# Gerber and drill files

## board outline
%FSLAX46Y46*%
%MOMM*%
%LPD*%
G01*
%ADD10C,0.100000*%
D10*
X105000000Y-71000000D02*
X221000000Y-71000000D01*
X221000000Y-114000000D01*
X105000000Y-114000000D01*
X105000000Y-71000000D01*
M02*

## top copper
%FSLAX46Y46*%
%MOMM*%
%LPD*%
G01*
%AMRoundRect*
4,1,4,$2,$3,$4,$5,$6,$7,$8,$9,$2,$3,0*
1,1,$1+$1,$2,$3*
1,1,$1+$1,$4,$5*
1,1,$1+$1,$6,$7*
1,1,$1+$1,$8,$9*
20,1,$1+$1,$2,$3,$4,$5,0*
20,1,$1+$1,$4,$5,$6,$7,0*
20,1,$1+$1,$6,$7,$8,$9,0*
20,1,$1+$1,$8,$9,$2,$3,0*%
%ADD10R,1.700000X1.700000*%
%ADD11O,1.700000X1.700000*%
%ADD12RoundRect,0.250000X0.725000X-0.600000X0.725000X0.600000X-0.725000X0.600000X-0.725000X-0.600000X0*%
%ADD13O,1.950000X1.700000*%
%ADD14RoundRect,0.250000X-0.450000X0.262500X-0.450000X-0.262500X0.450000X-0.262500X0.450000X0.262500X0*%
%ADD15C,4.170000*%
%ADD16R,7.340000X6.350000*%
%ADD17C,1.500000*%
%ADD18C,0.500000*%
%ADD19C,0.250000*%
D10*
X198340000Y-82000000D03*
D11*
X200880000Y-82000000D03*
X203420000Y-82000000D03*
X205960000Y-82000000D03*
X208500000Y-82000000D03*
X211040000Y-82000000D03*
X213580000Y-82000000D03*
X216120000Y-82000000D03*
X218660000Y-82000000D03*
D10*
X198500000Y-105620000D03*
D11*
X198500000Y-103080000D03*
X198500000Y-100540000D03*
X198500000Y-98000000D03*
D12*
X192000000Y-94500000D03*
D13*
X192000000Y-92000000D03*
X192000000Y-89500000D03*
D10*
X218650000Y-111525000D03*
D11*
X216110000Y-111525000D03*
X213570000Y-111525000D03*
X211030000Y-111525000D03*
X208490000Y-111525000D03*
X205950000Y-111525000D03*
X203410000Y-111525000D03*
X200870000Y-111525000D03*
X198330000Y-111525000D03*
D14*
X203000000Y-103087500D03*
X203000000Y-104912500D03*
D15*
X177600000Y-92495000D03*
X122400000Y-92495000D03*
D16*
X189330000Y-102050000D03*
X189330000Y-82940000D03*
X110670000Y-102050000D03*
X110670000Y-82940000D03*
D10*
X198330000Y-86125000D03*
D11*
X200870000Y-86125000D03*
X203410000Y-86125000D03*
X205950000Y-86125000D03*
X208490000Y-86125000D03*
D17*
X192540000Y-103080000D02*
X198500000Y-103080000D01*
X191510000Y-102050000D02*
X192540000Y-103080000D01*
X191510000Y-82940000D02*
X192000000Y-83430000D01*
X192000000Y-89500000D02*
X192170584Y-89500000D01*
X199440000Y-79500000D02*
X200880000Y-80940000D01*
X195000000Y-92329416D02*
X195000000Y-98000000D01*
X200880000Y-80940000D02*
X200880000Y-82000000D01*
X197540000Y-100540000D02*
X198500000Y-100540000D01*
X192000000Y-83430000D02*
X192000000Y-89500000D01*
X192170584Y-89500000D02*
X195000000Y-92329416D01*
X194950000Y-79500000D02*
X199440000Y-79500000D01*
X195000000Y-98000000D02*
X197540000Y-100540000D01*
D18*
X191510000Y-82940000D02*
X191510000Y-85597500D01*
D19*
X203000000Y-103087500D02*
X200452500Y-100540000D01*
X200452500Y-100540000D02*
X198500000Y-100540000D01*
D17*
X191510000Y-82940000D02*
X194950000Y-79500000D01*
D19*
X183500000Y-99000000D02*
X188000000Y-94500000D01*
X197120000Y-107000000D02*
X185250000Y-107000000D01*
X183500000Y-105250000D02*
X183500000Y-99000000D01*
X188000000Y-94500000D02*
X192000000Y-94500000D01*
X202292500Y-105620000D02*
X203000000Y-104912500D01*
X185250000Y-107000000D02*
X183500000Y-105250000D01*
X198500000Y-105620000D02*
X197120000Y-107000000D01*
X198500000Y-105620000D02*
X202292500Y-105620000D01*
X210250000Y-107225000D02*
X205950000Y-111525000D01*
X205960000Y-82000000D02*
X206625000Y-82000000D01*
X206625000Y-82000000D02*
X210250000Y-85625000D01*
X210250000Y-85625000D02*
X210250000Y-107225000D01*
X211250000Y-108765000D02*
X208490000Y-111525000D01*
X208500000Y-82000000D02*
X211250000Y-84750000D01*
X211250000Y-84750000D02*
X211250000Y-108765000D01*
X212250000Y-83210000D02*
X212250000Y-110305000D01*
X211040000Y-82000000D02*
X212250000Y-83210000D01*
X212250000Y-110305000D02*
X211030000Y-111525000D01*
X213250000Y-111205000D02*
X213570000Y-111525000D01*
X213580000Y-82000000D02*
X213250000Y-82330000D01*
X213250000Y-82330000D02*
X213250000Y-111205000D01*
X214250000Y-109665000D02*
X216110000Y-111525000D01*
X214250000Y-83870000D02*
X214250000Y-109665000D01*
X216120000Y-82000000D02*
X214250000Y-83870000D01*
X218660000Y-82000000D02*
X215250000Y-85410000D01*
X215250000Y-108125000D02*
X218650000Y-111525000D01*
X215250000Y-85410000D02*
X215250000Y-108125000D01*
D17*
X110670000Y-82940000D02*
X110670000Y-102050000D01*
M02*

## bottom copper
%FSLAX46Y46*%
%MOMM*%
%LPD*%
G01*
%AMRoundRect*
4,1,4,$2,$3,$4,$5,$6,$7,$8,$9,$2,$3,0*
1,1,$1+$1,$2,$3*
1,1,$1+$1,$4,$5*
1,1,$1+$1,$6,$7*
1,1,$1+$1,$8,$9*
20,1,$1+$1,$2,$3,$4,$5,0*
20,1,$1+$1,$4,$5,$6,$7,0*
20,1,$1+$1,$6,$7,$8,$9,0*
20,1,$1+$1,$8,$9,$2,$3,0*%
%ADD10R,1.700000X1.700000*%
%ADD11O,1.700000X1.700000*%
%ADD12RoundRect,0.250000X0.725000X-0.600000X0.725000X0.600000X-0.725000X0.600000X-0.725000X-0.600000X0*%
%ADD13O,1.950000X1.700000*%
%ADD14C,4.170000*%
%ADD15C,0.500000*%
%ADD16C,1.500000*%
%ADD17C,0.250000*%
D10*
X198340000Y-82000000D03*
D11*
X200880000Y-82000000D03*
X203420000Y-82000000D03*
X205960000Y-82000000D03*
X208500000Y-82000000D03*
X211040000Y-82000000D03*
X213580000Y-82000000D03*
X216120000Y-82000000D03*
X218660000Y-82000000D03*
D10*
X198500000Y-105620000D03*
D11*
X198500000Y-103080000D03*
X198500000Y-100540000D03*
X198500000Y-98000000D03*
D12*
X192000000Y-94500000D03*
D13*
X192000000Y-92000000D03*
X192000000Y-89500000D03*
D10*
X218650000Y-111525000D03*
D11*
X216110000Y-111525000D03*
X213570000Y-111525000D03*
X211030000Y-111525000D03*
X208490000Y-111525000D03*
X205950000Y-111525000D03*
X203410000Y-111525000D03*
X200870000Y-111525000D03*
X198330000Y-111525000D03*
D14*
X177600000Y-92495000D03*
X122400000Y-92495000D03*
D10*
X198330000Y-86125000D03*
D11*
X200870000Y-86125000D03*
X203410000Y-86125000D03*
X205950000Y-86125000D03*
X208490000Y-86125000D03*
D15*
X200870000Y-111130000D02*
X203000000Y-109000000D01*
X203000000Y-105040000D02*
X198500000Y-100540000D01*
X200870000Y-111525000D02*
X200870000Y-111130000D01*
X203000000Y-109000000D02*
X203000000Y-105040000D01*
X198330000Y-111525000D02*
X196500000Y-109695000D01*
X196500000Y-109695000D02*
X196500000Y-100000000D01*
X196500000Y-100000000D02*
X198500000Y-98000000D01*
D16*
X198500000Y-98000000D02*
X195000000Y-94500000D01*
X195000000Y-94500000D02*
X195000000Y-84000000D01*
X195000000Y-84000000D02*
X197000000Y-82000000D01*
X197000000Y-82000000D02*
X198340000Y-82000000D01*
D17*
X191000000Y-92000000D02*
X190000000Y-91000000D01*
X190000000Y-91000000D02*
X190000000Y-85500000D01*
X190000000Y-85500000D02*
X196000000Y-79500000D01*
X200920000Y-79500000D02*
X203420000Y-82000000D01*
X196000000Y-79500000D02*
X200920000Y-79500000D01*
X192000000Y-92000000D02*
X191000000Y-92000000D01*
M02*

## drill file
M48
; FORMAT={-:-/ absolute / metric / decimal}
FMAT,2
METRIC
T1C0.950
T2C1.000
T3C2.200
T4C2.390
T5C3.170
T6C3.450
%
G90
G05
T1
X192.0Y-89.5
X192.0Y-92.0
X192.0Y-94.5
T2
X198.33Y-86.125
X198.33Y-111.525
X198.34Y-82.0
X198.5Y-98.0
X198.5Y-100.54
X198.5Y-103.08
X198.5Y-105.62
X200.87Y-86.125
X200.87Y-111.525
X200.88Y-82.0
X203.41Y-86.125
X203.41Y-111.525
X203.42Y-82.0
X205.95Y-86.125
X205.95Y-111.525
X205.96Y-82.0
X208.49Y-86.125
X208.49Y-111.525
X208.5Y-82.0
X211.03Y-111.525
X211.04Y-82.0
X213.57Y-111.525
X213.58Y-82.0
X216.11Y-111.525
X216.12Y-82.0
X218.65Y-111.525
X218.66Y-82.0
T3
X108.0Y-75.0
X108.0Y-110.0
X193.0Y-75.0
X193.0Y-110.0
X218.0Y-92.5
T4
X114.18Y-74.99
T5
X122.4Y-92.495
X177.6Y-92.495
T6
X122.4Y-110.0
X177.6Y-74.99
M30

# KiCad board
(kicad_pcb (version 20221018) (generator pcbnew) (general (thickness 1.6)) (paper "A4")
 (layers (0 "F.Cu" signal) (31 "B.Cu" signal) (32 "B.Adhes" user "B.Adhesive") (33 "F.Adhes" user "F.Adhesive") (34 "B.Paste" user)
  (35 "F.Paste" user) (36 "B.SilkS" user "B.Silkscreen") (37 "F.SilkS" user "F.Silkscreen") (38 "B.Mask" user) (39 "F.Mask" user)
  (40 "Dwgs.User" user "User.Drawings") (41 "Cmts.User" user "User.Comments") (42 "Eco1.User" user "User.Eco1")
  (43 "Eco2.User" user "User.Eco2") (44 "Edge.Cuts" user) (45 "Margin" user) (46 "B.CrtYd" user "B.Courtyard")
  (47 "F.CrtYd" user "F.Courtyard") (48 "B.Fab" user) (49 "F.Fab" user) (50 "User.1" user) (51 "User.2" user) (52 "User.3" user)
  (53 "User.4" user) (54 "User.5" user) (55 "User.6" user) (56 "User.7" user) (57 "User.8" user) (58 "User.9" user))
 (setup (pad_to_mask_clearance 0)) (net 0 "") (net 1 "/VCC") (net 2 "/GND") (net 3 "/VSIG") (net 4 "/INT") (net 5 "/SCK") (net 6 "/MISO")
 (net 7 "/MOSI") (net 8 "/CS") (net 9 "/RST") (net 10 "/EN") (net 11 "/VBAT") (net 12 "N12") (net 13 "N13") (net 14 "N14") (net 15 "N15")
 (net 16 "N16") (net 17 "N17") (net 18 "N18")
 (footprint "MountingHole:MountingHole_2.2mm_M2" (layer "F.Cu") (at 108 110)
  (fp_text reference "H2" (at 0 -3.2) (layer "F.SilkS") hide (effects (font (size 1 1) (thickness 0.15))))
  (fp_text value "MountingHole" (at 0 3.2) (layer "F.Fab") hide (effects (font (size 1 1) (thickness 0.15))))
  (pad "" np_thru_hole circle (at 0 0) (size 2.2 2.2) (drill 2.2) (layers "*.Cu" "*.Mask")))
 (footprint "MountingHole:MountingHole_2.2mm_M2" (layer "F.Cu") (at 218 92.5)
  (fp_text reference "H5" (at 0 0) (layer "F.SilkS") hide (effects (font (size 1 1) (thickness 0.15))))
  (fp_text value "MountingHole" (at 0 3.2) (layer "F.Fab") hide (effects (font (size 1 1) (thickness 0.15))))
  (pad "" np_thru_hole circle (at 0 0) (size 2.2 2.2) (drill 2.2) (layers "*.Cu" "*.Mask")))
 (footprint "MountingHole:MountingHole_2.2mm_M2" (layer "F.Cu") (at 108 75)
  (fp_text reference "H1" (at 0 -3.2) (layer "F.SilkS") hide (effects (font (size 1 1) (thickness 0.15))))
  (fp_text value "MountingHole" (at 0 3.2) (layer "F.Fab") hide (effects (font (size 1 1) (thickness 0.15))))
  (pad "" np_thru_hole circle (at 0 0) (size 2.2 2.2) (drill 2.2) (layers "*.Cu" "*.Mask")))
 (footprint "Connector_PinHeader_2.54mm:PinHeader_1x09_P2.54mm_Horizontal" (layer "F.Cu") (at 198.34 82 90)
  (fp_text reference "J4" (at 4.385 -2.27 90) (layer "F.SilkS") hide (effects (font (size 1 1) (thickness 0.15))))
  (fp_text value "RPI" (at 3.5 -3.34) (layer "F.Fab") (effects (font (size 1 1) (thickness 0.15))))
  (pad "1" thru_hole rect (at 0 0 90) (size 1.7 1.7) (drill 1) (layers "*.Cu" "*.Mask") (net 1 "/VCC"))
  (pad "2" thru_hole oval (at 0 2.54 90) (size 1.7 1.7) (drill 1) (layers "*.Cu" "*.Mask") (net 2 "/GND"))
  (pad "3" thru_hole oval (at 0 5.08 90) (size 1.7 1.7) (drill 1) (layers "*.Cu" "*.Mask") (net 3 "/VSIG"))
  (pad "4" thru_hole oval (at 0 7.62 90) (size 1.7 1.7) (drill 1) (layers "*.Cu" "*.Mask") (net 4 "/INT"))
  (pad "5" thru_hole oval (at 0 10.16 90) (size 1.7 1.7) (drill 1) (layers "*.Cu" "*.Mask") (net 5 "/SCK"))
  (pad "6" thru_hole oval (at 0 12.7 90) (size 1.7 1.7) (drill 1) (layers "*.Cu" "*.Mask") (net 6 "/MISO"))
  (pad "7" thru_hole oval (at 0 15.24 90) (size 1.7 1.7) (drill 1) (layers "*.Cu" "*.Mask") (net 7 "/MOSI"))
  (pad "8" thru_hole oval (at 0 17.78 90) (size 1.7 1.7) (drill 1) (layers "*.Cu" "*.Mask") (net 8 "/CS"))
  (pad "9" thru_hole oval (at 0 20.32 90) (size 1.7 1.7) (drill 1) (layers "*.Cu" "*.Mask") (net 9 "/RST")))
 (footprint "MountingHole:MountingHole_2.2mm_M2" (layer "F.Cu") (at 193 110)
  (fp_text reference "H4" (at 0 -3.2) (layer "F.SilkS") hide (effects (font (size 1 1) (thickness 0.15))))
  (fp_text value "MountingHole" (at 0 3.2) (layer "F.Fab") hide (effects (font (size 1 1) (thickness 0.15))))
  (pad "" np_thru_hole circle (at 0 0) (size 2.2 2.2) (drill 2.2) (layers "*.Cu" "*.Mask")))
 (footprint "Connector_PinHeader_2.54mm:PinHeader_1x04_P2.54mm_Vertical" (layer "F.Cu") (at 198.5 105.62 180)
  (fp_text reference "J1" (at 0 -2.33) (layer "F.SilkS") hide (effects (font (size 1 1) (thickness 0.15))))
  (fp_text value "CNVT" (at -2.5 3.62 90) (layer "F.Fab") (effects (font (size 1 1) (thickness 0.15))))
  (pad "1" thru_hole rect (at 0 0 180) (size 1.7 1.7) (drill 1) (layers "*.Cu" "*.Mask") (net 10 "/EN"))
  (pad "2" thru_hole oval (at 0 2.54 180) (size 1.7 1.7) (drill 1) (layers "*.Cu" "*.Mask") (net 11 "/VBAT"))
  (pad "3" thru_hole oval (at 0 5.08 180) (size 1.7 1.7) (drill 1) (layers "*.Cu" "*.Mask") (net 2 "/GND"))
  (pad "4" thru_hole oval (at 0 7.62 180) (size 1.7 1.7) (drill 1) (layers "*.Cu" "*.Mask") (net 1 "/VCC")))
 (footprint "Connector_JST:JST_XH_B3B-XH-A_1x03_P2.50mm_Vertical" (layer "F.Cu") (at 192 94.5 90)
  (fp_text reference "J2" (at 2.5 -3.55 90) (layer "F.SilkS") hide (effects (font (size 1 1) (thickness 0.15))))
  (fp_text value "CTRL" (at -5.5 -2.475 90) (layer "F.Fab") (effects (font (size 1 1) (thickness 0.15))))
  (pad "1" thru_hole roundrect (at 0 0 90) (size 1.7 1.95) (drill 0.95) (layers "*.Cu" "*.Mask") (roundrect_rratio 0.1470588235)
   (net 10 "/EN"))
  (pad "2" thru_hole oval (at 2.5 0 90) (size 1.7 1.95) (drill 0.95) (layers "*.Cu" "*.Mask") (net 3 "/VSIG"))
  (pad "3" thru_hole oval (at 5 0 90) (size 1.7 1.95) (drill 0.95) (layers "*.Cu" "*.Mask") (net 2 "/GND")))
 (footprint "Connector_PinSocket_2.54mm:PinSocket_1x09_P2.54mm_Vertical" (layer "F.Cu") (at 218.65 111.525 -90)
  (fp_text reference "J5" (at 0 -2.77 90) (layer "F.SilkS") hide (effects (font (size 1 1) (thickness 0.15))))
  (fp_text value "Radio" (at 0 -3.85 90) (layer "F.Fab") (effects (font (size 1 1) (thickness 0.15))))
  (pad "1" thru_hole rect (at 0 0 270) (size 1.7 1.7) (drill 1) (layers "*.Cu" "*.Mask") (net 9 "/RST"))
  (pad "2" thru_hole oval (at 0 2.54 270) (size 1.7 1.7) (drill 1) (layers "*.Cu" "*.Mask") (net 8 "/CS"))
  (pad "3" thru_hole oval (at 0 5.08 270) (size 1.7 1.7) (drill 1) (layers "*.Cu" "*.Mask") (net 7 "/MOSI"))
  (pad "4" thru_hole oval (at 0 7.62 270) (size 1.7 1.7) (drill 1) (layers "*.Cu" "*.Mask") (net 6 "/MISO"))
  (pad "5" thru_hole oval (at 0 10.16 270) (size 1.7 1.7) (drill 1) (layers "*.Cu" "*.Mask") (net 5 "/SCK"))
  (pad "6" thru_hole oval (at 0 12.7 270) (size 1.7 1.7) (drill 1) (layers "*.Cu" "*.Mask") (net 4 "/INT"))
  (pad "7" thru_hole oval (at 0 15.24 270) (size 1.7 1.7) (drill 1) (layers "*.Cu" "*.Mask") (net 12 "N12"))
  (pad "8" thru_hole oval (at 0 17.78 270) (size 1.7 1.7) (drill 1) (layers "*.Cu" "*.Mask") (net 2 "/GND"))
  (pad "9" thru_hole oval (at 0 20.32 270) (size 1.7 1.7) (drill 1) (layers "*.Cu" "*.Mask") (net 1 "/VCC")))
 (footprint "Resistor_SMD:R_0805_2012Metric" (layer "F.Cu") (at 203 104 -90)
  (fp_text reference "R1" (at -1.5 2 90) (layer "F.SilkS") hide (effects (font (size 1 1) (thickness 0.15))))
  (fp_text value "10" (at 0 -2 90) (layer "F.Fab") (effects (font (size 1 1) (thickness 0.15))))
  (pad "1" smd roundrect (at -0.9125 0 270) (size 1.025 1.4) (layers "F.Cu" "F.Paste" "F.Mask") (roundrect_rratio 0.243902439)
   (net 2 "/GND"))
  (pad "2" smd roundrect (at 0.9125 0 270) (size 1.025 1.4) (layers "F.Cu" "F.Paste" "F.Mask") (roundrect_rratio 0.243902439) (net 10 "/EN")))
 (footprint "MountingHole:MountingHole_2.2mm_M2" (layer "F.Cu") (at 193 75)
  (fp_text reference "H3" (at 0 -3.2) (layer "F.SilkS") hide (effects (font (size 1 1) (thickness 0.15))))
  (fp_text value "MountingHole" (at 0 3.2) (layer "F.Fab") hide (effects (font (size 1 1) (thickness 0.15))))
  (pad "" np_thru_hole circle (at 0 0) (size 2.2 2.2) (drill 2.2) (layers "*.Cu" "*.Mask")))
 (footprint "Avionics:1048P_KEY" (layer "F.Cu") (at 150 92.495 180)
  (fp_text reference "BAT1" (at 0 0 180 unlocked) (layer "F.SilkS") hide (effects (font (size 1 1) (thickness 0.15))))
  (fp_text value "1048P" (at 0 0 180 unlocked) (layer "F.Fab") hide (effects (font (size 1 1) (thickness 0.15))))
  (pad "" np_thru_hole circle (at -27.6 0 180) (size 4.17 4.17) (drill 3.17) (layers "F&B.Cu" "*.Mask"))
  (pad "" np_thru_hole circle (at -27.6 17.505 180) (size 3.45 3.45) (drill 3.45) (layers "F&B.Cu" "*.Mask"))
  (pad "" np_thru_hole circle (at 27.6 -17.505 180) (size 3.45 3.45) (drill 3.45) (layers "F&B.Cu" "*.Mask"))
  (pad "" np_thru_hole circle (at 27.6 0 180) (size 4.17 4.17) (drill 3.17) (layers "F&B.Cu" "*.Mask"))
  (pad "" np_thru_hole circle (at 35.82 17.505 180) (size 2.39 2.39) (drill 2.39) (layers "F&B.Cu" "*.Mask"))
  (pad "1" smd rect (at -39.33 -9.555 180) (size 7.34 6.35) (layers "F.Cu" "F.Paste" "F.Mask") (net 11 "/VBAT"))
  (pad "2" smd rect (at -39.33 9.555 180) (size 7.34 6.35) (layers "F.Cu" "F.Paste" "F.Mask") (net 2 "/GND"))
  (pad "3" smd rect (at 39.33 -9.555 180) (size 7.34 6.35) (layers "F.Cu" "F.Paste" "F.Mask") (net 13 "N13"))
  (pad "4" smd rect (at 39.33 9.555 180) (size 7.34 6.35) (layers "F.Cu" "F.Paste" "F.Mask") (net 13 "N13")))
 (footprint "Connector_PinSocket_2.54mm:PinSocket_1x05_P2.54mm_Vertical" (layer "F.Cu") (at 198.33 86.125 90)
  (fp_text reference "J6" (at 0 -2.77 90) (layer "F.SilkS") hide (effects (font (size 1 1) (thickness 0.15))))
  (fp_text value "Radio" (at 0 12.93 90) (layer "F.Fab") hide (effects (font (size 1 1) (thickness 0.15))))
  (pad "1" thru_hole rect (at 0 0 90) (size 1.7 1.7) (drill 1) (layers "*.Cu" "*.Mask") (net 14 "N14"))
  (pad "2" thru_hole oval (at 0 2.54 90) (size 1.7 1.7) (drill 1) (layers "*.Cu" "*.Mask") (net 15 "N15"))
  (pad "3" thru_hole oval (at 0 5.08 90) (size 1.7 1.7) (drill 1) (layers "*.Cu" "*.Mask") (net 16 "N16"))
  (pad "4" thru_hole oval (at 0 7.62 90) (size 1.7 1.7) (drill 1) (layers "*.Cu" "*.Mask") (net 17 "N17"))
  (pad "5" thru_hole oval (at 0 10.16 90) (size 1.7 1.7) (drill 1) (layers "*.Cu" "*.Mask") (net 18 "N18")))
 (gr_rect (start 105 71) (end 221 114) (stroke (width 0.1) (type default)) (fill none) (layer "Edge.Cuts"))
 (segment (start 192.54 103.08) (end 198.5 103.08) (width 1.5) (layer "F.Cu") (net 11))
 (segment (start 191.51 102.05) (end 192.54 103.08) (width 1.5) (layer "F.Cu") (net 11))
 (segment (start 191.51 82.94) (end 192 83.43) (width 1.5) (layer "F.Cu") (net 2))
 (segment (start 192 89.5) (end 192.170584 89.5) (width 1.5) (layer "F.Cu") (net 2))
 (segment (start 199.44 79.5) (end 200.88 80.94) (width 1.5) (layer "F.Cu") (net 2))
 (segment (start 195 92.329416) (end 195 98) (width 1.5) (layer "F.Cu") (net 2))
 (segment (start 200.88 80.94) (end 200.88 82) (width 1.5) (layer "F.Cu") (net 2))
 (segment (start 197.54 100.54) (end 198.5 100.54) (width 1.5) (layer "F.Cu") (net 2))
 (segment (start 192 83.43) (end 192 89.5) (width 1.5) (layer "F.Cu") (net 2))
 (segment (start 192.170584 89.5) (end 195 92.329416) (width 1.5) (layer "F.Cu") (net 2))
 (segment (start 194.95 79.5) (end 199.44 79.5) (width 1.5) (layer "F.Cu") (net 2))
 (segment (start 195 98) (end 197.54 100.54) (width 1.5) (layer "F.Cu") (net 2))
 (segment (start 191.51 82.94) (end 191.51 85.5975) (width 0.5) (layer "F.Cu") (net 2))
 (segment (start 203 103.0875) (end 200.4525 100.54) (width 0.25) (layer "F.Cu") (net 2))
 (segment (start 200.4525 100.54) (end 198.5 100.54) (width 0.25) (layer "F.Cu") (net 2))
 (segment (start 191.51 82.94) (end 194.95 79.5) (width 1.5) (layer "F.Cu") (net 2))
 (segment (start 200.87 111.13) (end 203 109) (width 0.5) (layer "B.Cu") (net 2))
 (segment (start 203 105.04) (end 198.5 100.54) (width 0.5) (layer "B.Cu") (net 2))
 (segment (start 200.87 111.525) (end 200.87 111.13) (width 0.5) (layer "B.Cu") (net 2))
 (segment (start 203 109) (end 203 105.04) (width 0.5) (layer "B.Cu") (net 2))
 (segment (start 183.5 99) (end 188 94.5) (width 0.25) (layer "F.Cu") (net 10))
 (segment (start 197.12 107) (end 185.25 107) (width 0.25) (layer "F.Cu") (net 10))
 (segment (start 183.5 105.25) (end 183.5 99) (width 0.25) (layer "F.Cu") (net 10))
 (segment (start 188 94.5) (end 192 94.5) (width 0.25) (layer "F.Cu") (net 10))
 (segment (start 202.2925 105.62) (end 203 104.9125) (width 0.25) (layer "F.Cu") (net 10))
 (segment (start 185.25 107) (end 183.5 105.25) (width 0.25) (layer "F.Cu") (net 10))
 (segment (start 198.5 105.62) (end 197.12 107) (width 0.25) (layer "F.Cu") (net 10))
 (segment (start 198.5 105.62) (end 202.2925 105.62) (width 0.25) (layer "F.Cu") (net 10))
 (segment (start 198.33 111.525) (end 196.5 109.695) (width 0.5) (layer "B.Cu") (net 1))
 (segment (start 196.5 109.695) (end 196.5 100) (width 0.5) (layer "B.Cu") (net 1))
 (segment (start 196.5 100) (end 198.5 98) (width 0.5) (layer "B.Cu") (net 1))
 (segment (start 198.5 98) (end 195 94.5) (width 1.5) (layer "B.Cu") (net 1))
 (segment (start 195 94.5) (end 195 84) (width 1.5) (layer "B.Cu") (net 1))
 (segment (start 195 84) (end 197 82) (width 1.5) (layer "B.Cu") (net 1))
 (segment (start 197 82) (end 198.34 82) (width 1.5) (layer "B.Cu") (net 1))
 (segment (start 191 92) (end 190 91) (width 0.25) (layer "B.Cu") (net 3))
 (segment (start 190 91) (end 190 85.5) (width 0.25) (layer "B.Cu") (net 3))
 (segment (start 190 85.5) (end 196 79.5) (width 0.25) (layer "B.Cu") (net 3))
 (segment (start 200.92 79.5) (end 203.42 82) (width 0.25) (layer "B.Cu") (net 3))
 (segment (start 196 79.5) (end 200.92 79.5) (width 0.25) (layer "B.Cu") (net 3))
 (segment (start 192 92) (end 191 92) (width 0.25) (layer "B.Cu") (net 3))
 (segment (start 210.25 107.225) (end 205.95 111.525) (width 0.25) (layer "F.Cu") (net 4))
 (segment (start 205.96 82) (end 206.625 82) (width 0.25) (layer "F.Cu") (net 4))
 (segment (start 206.625 82) (end 210.25 85.625) (width 0.25) (layer "F.Cu") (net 4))
 (segment (start 210.25 85.625) (end 210.25 107.225) (width 0.25) (layer "F.Cu") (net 4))
 (segment (start 211.25 108.765) (end 208.49 111.525) (width 0.25) (layer "F.Cu") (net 5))
 (segment (start 208.5 82) (end 211.25 84.75) (width 0.25) (layer "F.Cu") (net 5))
 (segment (start 211.25 84.75) (end 211.25 108.765) (width 0.25) (layer "F.Cu") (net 5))
 (segment (start 212.25 83.21) (end 212.25 110.305) (width 0.25) (layer "F.Cu") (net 6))
 (segment (start 211.04 82) (end 212.25 83.21) (width 0.25) (layer "F.Cu") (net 6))
 (segment (start 212.25 110.305) (end 211.03 111.525) (width 0.25) (layer "F.Cu") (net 6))
 (segment (start 213.25 111.205) (end 213.57 111.525) (width 0.25) (layer "F.Cu") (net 7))
 (segment (start 213.58 82) (end 213.25 82.33) (width 0.25) (layer "F.Cu") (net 7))
 (segment (start 213.25 82.33) (end 213.25 111.205) (width 0.25) (layer "F.Cu") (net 7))
 (segment (start 214.25 109.665) (end 216.11 111.525) (width 0.25) (layer "F.Cu") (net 8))
 (segment (start 214.25 83.87) (end 214.25 109.665) (width 0.25) (layer "F.Cu") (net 8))
 (segment (start 216.12 82) (end 214.25 83.87) (width 0.25) (layer "F.Cu") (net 8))
 (segment (start 218.66 82) (end 215.25 85.41) (width 0.25) (layer "F.Cu") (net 9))
 (segment (start 215.25 108.125) (end 218.65 111.525) (width 0.25) (layer "F.Cu") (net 9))
 (segment (start 215.25 85.41) (end 215.25 108.125) (width 0.25) (layer "F.Cu") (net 9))
 (segment (start 110.67 82.94) (end 110.67 102.05) (width 1.5) (layer "F.Cu") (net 13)))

